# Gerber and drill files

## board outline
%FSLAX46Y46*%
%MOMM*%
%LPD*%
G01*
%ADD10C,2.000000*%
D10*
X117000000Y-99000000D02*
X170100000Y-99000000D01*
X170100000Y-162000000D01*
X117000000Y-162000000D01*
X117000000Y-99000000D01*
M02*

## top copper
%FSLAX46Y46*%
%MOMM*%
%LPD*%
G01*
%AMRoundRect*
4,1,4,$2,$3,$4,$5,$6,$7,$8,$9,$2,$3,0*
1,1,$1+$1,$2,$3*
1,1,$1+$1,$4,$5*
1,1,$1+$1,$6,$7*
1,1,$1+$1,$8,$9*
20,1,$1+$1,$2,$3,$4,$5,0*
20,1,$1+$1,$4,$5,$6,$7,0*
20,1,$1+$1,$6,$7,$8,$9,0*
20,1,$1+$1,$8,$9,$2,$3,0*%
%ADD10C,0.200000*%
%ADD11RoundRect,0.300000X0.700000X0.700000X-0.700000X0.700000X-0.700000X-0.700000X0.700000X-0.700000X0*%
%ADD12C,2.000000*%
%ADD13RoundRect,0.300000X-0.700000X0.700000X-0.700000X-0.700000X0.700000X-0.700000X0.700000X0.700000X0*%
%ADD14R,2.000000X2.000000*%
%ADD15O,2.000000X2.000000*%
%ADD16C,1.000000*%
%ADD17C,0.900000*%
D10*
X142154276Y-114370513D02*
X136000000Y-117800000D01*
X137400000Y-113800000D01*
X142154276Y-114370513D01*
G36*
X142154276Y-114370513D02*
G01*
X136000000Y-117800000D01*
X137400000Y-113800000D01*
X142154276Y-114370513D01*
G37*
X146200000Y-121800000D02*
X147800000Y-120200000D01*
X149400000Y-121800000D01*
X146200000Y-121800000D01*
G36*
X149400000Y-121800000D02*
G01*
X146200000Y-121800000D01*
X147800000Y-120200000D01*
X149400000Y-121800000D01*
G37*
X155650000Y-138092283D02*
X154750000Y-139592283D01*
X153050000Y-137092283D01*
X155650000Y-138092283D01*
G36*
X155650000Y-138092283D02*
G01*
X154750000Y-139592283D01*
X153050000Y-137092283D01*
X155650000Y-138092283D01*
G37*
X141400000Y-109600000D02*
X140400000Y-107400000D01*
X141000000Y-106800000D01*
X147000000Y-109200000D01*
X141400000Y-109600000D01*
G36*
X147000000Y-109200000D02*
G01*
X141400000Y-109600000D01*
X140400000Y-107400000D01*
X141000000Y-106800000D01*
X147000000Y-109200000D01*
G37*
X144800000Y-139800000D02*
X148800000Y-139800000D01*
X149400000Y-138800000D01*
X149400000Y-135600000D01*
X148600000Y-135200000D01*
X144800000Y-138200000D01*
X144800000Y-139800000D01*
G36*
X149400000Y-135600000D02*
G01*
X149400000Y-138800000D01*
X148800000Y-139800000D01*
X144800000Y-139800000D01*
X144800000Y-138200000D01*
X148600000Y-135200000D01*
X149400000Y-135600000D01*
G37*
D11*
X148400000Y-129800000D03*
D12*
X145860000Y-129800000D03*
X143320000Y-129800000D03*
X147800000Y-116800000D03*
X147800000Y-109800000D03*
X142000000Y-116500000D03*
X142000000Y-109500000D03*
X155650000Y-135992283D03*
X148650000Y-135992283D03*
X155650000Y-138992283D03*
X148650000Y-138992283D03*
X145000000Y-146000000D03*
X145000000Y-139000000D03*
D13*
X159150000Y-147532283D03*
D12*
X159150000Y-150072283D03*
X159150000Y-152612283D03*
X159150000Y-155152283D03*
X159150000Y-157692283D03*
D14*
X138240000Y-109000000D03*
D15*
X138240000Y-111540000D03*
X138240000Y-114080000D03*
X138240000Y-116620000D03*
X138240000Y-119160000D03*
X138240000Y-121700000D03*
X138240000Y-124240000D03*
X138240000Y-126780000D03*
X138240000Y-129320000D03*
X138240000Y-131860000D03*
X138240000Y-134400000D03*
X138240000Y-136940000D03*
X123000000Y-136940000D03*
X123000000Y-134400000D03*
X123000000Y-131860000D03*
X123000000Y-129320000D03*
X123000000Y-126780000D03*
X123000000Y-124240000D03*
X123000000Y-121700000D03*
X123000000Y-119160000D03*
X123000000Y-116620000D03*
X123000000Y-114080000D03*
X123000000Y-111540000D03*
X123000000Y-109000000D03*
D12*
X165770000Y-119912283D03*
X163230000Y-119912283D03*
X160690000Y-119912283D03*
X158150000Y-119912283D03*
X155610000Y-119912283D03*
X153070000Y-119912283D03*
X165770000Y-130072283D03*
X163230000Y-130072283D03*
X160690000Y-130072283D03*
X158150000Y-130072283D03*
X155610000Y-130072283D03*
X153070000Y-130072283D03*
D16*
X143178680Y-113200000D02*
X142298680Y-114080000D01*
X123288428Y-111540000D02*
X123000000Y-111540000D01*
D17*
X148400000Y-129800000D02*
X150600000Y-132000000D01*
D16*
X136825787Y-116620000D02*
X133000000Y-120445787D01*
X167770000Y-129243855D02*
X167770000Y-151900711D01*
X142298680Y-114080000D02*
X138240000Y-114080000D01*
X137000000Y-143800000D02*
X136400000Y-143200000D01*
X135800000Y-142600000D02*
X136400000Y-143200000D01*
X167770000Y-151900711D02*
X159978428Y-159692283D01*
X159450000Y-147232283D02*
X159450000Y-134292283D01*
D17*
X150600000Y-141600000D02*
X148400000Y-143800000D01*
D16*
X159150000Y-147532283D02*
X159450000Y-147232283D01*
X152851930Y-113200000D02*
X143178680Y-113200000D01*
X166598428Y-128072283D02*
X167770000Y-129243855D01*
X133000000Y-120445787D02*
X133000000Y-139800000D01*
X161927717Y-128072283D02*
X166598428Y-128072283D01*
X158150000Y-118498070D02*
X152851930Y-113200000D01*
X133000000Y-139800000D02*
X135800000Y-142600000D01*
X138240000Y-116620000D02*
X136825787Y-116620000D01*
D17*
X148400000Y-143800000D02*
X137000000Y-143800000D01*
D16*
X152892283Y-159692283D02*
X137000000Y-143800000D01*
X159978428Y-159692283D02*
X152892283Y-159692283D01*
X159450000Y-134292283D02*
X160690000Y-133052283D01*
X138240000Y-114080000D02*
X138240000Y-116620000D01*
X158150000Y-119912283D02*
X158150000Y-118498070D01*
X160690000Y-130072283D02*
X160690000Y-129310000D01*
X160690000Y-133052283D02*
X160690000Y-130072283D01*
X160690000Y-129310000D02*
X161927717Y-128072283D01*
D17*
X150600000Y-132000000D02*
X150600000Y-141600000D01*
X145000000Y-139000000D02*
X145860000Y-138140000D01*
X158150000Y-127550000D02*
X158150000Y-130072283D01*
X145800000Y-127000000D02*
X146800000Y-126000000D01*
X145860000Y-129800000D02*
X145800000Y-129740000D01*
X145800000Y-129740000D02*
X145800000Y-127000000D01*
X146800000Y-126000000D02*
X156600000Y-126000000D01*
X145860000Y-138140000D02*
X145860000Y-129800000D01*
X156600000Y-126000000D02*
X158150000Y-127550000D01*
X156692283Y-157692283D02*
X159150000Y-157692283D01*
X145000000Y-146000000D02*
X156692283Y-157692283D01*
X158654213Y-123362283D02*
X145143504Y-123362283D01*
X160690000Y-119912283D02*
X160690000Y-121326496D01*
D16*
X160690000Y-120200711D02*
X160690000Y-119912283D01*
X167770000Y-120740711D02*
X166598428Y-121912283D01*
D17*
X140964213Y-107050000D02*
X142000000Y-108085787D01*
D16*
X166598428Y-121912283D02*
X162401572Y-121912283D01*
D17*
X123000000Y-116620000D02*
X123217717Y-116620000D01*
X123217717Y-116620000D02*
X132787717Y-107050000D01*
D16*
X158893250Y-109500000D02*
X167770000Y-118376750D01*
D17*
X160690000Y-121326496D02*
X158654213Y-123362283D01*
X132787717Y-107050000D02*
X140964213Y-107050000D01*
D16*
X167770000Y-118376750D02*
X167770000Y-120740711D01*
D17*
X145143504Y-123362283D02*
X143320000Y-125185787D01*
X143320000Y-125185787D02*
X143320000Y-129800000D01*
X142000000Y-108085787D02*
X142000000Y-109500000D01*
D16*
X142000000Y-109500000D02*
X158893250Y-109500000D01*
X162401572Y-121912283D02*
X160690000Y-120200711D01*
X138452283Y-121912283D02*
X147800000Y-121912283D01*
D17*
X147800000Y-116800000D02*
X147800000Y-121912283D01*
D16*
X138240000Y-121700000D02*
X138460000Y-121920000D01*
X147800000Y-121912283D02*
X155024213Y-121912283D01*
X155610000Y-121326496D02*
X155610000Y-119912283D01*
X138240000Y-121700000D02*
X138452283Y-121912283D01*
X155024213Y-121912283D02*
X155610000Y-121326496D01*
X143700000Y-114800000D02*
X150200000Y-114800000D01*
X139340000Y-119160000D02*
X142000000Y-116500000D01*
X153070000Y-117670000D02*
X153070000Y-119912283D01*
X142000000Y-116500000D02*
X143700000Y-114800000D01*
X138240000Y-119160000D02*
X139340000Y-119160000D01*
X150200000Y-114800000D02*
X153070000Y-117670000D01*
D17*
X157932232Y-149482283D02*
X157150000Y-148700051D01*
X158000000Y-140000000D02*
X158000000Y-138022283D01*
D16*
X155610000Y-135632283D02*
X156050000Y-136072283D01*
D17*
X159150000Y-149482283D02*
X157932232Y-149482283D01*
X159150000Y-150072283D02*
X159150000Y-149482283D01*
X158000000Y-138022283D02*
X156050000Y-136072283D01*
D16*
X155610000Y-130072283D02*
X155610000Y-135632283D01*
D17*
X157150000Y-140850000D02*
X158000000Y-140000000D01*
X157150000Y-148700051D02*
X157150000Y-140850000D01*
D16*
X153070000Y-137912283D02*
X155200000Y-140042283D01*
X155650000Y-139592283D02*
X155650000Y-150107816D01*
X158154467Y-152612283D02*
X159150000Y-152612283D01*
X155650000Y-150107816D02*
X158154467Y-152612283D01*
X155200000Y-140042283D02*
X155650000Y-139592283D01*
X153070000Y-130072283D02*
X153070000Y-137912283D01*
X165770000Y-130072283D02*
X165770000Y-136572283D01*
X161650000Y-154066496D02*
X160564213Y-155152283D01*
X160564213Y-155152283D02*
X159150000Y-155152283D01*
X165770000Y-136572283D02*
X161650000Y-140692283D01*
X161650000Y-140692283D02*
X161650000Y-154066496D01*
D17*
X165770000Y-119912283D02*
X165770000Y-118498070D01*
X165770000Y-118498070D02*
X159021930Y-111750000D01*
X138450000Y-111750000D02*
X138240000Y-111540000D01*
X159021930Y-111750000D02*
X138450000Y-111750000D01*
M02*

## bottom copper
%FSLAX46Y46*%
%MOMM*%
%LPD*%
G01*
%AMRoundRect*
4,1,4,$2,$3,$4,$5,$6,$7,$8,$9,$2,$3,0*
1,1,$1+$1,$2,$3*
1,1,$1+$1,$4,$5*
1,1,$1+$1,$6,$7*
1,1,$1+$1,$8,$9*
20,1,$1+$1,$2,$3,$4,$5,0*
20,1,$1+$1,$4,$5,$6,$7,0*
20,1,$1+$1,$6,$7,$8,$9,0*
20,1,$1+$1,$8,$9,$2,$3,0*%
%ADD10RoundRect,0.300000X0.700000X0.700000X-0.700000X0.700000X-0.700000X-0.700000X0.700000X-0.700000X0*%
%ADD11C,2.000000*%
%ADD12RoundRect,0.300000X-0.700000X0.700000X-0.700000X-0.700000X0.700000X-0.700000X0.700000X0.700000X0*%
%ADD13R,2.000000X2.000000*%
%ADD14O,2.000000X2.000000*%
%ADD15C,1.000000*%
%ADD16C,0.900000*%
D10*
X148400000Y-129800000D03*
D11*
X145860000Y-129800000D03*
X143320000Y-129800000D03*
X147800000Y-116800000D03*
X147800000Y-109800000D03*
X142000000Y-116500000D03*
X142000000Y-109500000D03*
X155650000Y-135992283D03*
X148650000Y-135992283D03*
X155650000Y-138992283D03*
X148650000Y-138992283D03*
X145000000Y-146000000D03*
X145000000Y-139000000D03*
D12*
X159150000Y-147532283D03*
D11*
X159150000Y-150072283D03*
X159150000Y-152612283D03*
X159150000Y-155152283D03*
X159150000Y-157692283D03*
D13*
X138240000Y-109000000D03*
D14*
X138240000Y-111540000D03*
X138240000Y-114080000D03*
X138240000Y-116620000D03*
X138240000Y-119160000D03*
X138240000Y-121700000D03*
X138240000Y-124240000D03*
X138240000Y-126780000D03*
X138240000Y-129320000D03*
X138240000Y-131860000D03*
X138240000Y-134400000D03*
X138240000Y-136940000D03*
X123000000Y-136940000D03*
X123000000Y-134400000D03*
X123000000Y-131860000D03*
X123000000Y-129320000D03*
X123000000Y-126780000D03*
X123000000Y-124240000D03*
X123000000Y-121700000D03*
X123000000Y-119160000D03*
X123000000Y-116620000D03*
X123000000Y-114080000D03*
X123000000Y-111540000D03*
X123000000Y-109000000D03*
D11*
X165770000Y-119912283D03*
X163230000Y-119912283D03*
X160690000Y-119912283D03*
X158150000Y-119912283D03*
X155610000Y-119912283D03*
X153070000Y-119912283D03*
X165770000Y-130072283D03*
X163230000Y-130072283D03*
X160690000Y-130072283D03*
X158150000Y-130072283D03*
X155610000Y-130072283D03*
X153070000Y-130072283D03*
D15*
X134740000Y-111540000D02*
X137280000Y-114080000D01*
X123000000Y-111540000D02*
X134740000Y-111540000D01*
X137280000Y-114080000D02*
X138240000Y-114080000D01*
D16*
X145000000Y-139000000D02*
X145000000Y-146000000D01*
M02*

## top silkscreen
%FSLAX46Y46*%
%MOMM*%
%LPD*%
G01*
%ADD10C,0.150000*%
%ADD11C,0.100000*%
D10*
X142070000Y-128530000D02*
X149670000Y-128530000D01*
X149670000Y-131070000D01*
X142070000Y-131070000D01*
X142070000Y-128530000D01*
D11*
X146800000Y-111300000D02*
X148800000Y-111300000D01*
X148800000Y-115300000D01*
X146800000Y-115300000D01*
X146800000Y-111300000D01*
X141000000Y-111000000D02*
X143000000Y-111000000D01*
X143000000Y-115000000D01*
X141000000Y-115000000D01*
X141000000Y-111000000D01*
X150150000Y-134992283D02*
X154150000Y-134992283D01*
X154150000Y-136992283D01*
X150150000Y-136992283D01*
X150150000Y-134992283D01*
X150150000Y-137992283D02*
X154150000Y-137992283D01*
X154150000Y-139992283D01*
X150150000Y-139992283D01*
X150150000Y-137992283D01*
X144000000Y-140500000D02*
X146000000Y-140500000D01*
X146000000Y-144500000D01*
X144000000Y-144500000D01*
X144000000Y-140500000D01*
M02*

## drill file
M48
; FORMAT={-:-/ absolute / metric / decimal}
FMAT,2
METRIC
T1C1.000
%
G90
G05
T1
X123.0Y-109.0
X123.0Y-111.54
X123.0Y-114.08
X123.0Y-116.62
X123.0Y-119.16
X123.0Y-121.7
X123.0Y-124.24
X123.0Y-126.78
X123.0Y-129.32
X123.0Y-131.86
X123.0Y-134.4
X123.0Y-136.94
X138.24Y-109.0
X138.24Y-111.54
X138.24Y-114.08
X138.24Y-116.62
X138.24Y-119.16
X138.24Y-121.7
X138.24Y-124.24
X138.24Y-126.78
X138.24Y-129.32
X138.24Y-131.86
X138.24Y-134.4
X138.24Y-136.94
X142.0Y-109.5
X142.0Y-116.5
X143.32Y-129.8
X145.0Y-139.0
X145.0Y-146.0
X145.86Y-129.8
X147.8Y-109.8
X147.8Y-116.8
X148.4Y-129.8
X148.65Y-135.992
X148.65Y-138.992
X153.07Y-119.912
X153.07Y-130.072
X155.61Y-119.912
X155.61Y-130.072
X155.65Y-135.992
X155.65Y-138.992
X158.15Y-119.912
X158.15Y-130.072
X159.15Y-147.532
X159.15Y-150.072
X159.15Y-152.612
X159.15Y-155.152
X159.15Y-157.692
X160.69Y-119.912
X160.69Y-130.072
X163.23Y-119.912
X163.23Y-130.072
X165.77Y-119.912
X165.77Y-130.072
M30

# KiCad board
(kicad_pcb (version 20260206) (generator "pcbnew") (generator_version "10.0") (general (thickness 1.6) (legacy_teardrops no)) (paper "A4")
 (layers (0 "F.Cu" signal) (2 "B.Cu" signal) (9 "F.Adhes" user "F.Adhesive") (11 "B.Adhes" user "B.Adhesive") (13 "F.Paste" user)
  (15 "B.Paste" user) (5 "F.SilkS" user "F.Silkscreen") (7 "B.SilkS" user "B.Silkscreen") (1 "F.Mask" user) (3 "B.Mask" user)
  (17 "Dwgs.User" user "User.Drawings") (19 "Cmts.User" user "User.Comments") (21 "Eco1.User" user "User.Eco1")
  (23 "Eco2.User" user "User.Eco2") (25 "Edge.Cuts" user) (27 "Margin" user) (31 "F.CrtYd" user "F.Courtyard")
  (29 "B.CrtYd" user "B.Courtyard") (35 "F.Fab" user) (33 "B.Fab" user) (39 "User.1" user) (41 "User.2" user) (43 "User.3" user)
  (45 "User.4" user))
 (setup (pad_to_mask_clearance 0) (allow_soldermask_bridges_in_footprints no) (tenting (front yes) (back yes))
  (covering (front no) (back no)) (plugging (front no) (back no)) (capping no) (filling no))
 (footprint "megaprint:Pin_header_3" (layer "F.Cu") (at 145.86 129.8 180)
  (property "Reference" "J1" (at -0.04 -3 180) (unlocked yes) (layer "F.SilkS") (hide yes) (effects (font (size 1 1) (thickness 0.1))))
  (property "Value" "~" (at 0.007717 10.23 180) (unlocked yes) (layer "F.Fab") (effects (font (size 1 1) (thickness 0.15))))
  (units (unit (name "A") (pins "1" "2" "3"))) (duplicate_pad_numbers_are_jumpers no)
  (fp_rect (start -3.81 -1.27) (end 3.79 1.27) (stroke (width 0.15) (type default)) (fill no) (layer "F.SilkS"))
  (pad "1" thru_hole roundrect (at -2.54 0 180) (size 2 2) (drill 1) (layers "*.Cu" "*.Mask") (remove_unused_layers no)
   (roundrect_rratio 0.15) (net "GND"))
  (pad "2" thru_hole circle (at 0 0 180) (size 2 2) (drill 1) (layers "*.Cu" "*.Mask") (remove_unused_layers no) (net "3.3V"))
  (pad "3" thru_hole circle (at 2.54 0 180) (size 2 2) (drill 1) (layers "*.Cu" "*.Mask") (remove_unused_layers no) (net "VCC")))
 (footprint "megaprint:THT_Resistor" (layer "F.Cu") (at 147.8 113.3 90)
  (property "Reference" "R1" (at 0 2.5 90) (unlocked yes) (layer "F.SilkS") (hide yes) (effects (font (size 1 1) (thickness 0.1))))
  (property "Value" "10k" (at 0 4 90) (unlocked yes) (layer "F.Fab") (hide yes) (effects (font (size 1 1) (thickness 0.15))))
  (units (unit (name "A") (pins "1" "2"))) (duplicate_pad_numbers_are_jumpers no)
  (fp_rect (start -2 -1) (end 2 1) (stroke (width 0.1) (type default)) (fill no) (layer "F.SilkS"))
  (pad "1" thru_hole circle (at -3.5 0 90) (size 2 2) (drill 1) (layers "*.Cu" "*.Mask") (remove_unused_layers no) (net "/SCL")
   (thermal_bridge_angle 90))
  (pad "2" thru_hole circle (at 3.5 0 90) (size 2 2) (drill 1) (layers "*.Cu" "*.Mask") (remove_unused_layers no) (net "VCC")
   (thermal_bridge_angle 90)))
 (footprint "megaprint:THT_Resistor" (layer "F.Cu") (at 142 113 90)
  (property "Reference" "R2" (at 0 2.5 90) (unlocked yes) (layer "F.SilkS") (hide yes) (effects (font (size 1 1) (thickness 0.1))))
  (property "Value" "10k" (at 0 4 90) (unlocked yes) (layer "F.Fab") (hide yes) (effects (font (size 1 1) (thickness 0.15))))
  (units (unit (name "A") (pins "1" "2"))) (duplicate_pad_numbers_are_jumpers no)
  (fp_rect (start -2 -1) (end 2 1) (stroke (width 0.1) (type default)) (fill no) (layer "F.SilkS"))
  (pad "1" thru_hole circle (at -3.5 0 90) (size 2 2) (drill 1) (layers "*.Cu" "*.Mask") (remove_unused_layers no) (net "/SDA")
   (thermal_bridge_angle 90))
  (pad "2" thru_hole circle (at 3.5 0 90) (size 2 2) (drill 1) (layers "*.Cu" "*.Mask") (remove_unused_layers no) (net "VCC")
   (thermal_bridge_angle 90)))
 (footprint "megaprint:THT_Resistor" (layer "F.Cu") (at 152.15 135.992283 180)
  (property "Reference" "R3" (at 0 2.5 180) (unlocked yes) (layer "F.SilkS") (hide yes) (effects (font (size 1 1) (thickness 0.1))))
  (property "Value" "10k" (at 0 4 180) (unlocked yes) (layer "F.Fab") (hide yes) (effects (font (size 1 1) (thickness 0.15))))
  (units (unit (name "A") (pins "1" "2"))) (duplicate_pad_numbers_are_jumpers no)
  (fp_rect (start -2 -1) (end 2 1) (stroke (width 0.1) (type default)) (fill no) (layer "F.SilkS"))
  (pad "1" thru_hole circle (at -3.5 0 180) (size 2 2) (drill 1) (layers "*.Cu" "*.Mask") (remove_unused_layers no) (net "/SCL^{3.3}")
   (thermal_bridge_angle 90))
  (pad "2" thru_hole circle (at 3.5 0 180) (size 2 2) (drill 1) (layers "*.Cu" "*.Mask") (remove_unused_layers no) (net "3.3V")
   (thermal_bridge_angle 90)))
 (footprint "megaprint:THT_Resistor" (layer "F.Cu") (at 152.15 138.992283 180)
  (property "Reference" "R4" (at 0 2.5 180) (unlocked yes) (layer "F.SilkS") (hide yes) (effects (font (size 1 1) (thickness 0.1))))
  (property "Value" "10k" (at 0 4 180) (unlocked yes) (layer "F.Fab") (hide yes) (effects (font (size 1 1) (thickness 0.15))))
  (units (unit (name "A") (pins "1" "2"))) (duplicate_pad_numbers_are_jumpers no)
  (fp_rect (start -2 -1) (end 2 1) (stroke (width 0.1) (type default)) (fill no) (layer "F.SilkS"))
  (pad "1" thru_hole circle (at -3.5 0 180) (size 2 2) (drill 1) (layers "*.Cu" "*.Mask") (remove_unused_layers no) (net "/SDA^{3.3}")
   (thermal_bridge_angle 90))
  (pad "2" thru_hole circle (at 3.5 0 180) (size 2 2) (drill 1) (layers "*.Cu" "*.Mask") (remove_unused_layers no) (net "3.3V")
   (thermal_bridge_angle 90)))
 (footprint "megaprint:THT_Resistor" (layer "F.Cu") (at 145 142.5 90)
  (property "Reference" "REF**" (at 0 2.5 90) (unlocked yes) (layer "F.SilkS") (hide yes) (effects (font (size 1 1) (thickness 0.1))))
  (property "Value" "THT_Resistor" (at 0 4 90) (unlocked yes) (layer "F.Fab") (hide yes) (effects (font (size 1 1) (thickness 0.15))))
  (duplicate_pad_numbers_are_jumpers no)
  (fp_rect (start -2 -1) (end 2 1) (stroke (width 0.1) (type default)) (fill no) (layer "F.SilkS"))
  (pad "1" thru_hole circle (at -3.5 0 90) (size 2 2) (drill 1) (layers "*.Cu" "*.Mask") (remove_unused_layers no) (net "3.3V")
   (thermal_bridge_angle 90))
  (pad "2" thru_hole circle (at 3.5 0 90) (size 2 2) (drill 1) (layers "*.Cu" "*.Mask") (remove_unused_layers no) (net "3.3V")
   (thermal_bridge_angle 90)))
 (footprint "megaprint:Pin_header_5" (layer "B.Cu") (at 159.15 152.612283 -90)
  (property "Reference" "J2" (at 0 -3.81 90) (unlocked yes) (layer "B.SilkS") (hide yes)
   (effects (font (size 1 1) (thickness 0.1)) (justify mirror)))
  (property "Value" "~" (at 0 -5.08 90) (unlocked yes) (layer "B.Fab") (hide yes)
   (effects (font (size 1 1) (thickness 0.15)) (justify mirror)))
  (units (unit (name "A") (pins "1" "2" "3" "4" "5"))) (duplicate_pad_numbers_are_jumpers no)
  (pad "1" thru_hole roundrect (at -5.08 0 270) (size 2 2) (drill 1) (layers "*.Cu" "*.Mask") (remove_unused_layers no)
   (roundrect_rratio 0.15) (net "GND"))
  (pad "2" thru_hole circle (at -2.54 0 270) (size 2 2) (drill 1) (layers "*.Cu" "*.Mask") (remove_unused_layers no) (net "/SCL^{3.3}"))
  (pad "3" thru_hole circle (at 0 0 270) (size 2 2) (drill 1) (layers "*.Cu" "*.Mask") (remove_unused_layers no) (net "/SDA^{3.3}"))
  (pad "4" thru_hole circle (at 2.54 0 270) (size 2 2) (drill 1) (layers "*.Cu" "*.Mask") (remove_unused_layers no) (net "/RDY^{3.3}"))
  (pad "5" thru_hole circle (at 5.08 0 270) (size 2 2) (drill 1) (layers "*.Cu" "*.Mask") (remove_unused_layers no) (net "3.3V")))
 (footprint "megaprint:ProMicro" (layer "B.Cu") (at 130.62 120.43 180)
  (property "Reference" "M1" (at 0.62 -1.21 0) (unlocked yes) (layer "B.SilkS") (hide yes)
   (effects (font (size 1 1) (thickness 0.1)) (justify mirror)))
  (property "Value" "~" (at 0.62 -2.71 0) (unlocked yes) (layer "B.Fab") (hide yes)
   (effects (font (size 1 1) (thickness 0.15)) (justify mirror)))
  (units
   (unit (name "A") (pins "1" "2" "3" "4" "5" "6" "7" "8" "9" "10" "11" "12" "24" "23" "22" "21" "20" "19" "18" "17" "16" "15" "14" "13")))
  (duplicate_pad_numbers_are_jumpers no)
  (pad "1" thru_hole rect (at -7.62 11.43) (size 2 2) (drill 1) (layers "*.Cu" "*.Mask") (remove_unused_layers no)
   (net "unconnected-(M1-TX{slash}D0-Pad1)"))
  (pad "2" thru_hole oval (at -7.62 8.89) (size 2 2) (drill 1) (layers "*.Cu" "*.Mask") (remove_unused_layers no) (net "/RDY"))
  (pad "3" thru_hole oval (at -7.62 6.35) (size 2 2) (drill 1) (layers "*.Cu" "*.Mask") (remove_unused_layers no) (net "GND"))
  (pad "4" thru_hole oval (at -7.62 3.81) (size 2 2) (drill 1) (layers "*.Cu" "*.Mask") (remove_unused_layers no) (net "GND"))
  (pad "5" thru_hole oval (at -7.62 1.27) (size 2 2) (drill 1) (layers "*.Cu" "*.Mask") (remove_unused_layers no) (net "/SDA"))
  (pad "6" thru_hole oval (at -7.62 -1.27) (size 2 2) (drill 1) (layers "*.Cu" "*.Mask") (remove_unused_layers no) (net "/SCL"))
  (pad "7" thru_hole oval (at -7.62 -3.81) (size 2 2) (drill 1) (layers "*.Cu" "*.Mask") (remove_unused_layers no)
   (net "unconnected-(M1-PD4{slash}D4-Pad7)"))
  (pad "8" thru_hole oval (at -7.62 -6.35) (size 2 2) (drill 1) (layers "*.Cu" "*.Mask") (remove_unused_layers no)
   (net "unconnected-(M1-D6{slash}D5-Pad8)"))
  (pad "9" thru_hole oval (at -7.62 -8.89) (size 2 2) (drill 1) (layers "*.Cu" "*.Mask") (remove_unused_layers no)
   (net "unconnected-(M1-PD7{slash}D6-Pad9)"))
  (pad "10" thru_hole oval (at -7.62 -11.43) (size 2 2) (drill 1) (layers "*.Cu" "*.Mask") (remove_unused_layers no)
   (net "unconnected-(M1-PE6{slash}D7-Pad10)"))
  (pad "11" thru_hole oval (at -7.62 -13.97) (size 2 2) (drill 1) (layers "*.Cu" "*.Mask") (remove_unused_layers no)
   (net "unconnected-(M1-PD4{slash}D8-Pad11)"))
  (pad "12" thru_hole oval (at -7.62 -16.51) (size 2 2) (drill 1) (layers "*.Cu" "*.Mask") (remove_unused_layers no)
   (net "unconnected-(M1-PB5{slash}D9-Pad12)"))
  (pad "13" thru_hole oval (at 7.62 -16.51) (size 2 2) (drill 1) (layers "*.Cu" "*.Mask") (remove_unused_layers no)
   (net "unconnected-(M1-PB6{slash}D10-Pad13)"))
  (pad "14" thru_hole oval (at 7.62 -13.97) (size 2 2) (drill 1) (layers "*.Cu" "*.Mask") (remove_unused_layers no)
   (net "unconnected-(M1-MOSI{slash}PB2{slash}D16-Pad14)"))
  (pad "15" thru_hole oval (at 7.62 -11.43) (size 2 2) (drill 1) (layers "*.Cu" "*.Mask") (remove_unused_layers no)
   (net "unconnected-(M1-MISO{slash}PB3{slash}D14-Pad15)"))
  (pad "16" thru_hole oval (at 7.62 -8.89) (size 2 2) (drill 1) (layers "*.Cu" "*.Mask") (remove_unused_layers no)
   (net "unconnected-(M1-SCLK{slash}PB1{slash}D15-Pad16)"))
  (pad "17" thru_hole oval (at 7.62 -6.35) (size 2 2) (drill 1) (layers "*.Cu" "*.Mask") (remove_unused_layers no)
   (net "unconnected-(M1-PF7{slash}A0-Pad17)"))
  (pad "18" thru_hole oval (at 7.62 -3.81) (size 2 2) (drill 1) (layers "*.Cu" "*.Mask") (remove_unused_layers no)
   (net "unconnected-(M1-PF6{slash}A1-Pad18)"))
  (pad "19" thru_hole oval (at 7.62 -1.27) (size 2 2) (drill 1) (layers "*.Cu" "*.Mask") (remove_unused_layers no)
   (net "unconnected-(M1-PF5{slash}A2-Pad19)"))
  (pad "20" thru_hole oval (at 7.62 1.27) (size 2 2) (drill 1) (layers "*.Cu" "*.Mask") (remove_unused_layers no)
   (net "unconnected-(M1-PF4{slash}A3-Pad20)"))
  (pad "21" thru_hole oval (at 7.62 3.81) (size 2 2) (drill 1) (layers "*.Cu" "*.Mask") (remove_unused_layers no) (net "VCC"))
  (pad "22" thru_hole oval (at 7.62 6.35) (size 2 2) (drill 1) (layers "*.Cu" "*.Mask") (remove_unused_layers no)
   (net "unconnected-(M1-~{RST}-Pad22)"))
  (pad "23" thru_hole oval (at 7.62 8.89) (size 2 2) (drill 1) (layers "*.Cu" "*.Mask") (remove_unused_layers no) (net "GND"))
  (pad "24" thru_hole oval (at 7.62 11.43) (size 2 2) (drill 1) (layers "*.Cu" "*.Mask") (remove_unused_layers no)
   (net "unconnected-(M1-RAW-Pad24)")))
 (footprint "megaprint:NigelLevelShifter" (layer "B.Cu") (at 159.4125 124.992283 180)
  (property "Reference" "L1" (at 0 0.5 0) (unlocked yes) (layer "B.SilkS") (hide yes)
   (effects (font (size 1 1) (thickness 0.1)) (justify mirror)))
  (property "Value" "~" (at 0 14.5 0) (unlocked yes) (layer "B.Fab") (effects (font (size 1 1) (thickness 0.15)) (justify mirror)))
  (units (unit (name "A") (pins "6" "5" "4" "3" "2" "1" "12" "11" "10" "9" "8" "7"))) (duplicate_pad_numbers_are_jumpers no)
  (pad "1" thru_hole circle (at -6.3575 5.08 180) (size 2 2) (drill 1) (layers "*.Cu" "*.Mask") (remove_unused_layers no) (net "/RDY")
   (thermal_bridge_angle 90))
  (pad "2" thru_hole circle (at -3.8175 5.08 180) (size 2 2) (drill 1) (layers "*.Cu" "*.Mask") (remove_unused_layers no)
   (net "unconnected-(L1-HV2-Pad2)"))
  (pad "3" thru_hole circle (at -1.2775 5.08 180) (size 2 2) (drill 1) (layers "*.Cu" "*.Mask") (remove_unused_layers no) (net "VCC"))
  (pad "4" thru_hole circle (at 1.2625 5.08 180) (size 2 2) (drill 1) (layers "*.Cu" "*.Mask") (remove_unused_layers no) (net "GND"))
  (pad "5" thru_hole circle (at 3.8025 5.08 180) (size 2 2) (drill 1) (layers "*.Cu" "*.Mask") (remove_unused_layers no) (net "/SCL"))
  (pad "6" thru_hole circle (at 6.3425 5.08 180) (size 2 2) (drill 1) (layers "*.Cu" "*.Mask") (remove_unused_layers no) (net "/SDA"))
  (pad "7" thru_hole circle (at -6.3575 -5.08 180) (size 2 2) (drill 1) (layers "*.Cu" "*.Mask") (remove_unused_layers no)
   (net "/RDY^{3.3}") (thermal_bridge_angle 90))
  (pad "8" thru_hole circle (at -3.8175 -5.08 180) (size 2 2) (drill 1) (layers "*.Cu" "*.Mask") (remove_unused_layers no)
   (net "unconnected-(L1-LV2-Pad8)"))
  (pad "9" thru_hole circle (at -1.2775 -5.08 180) (size 2 2) (drill 1) (layers "*.Cu" "*.Mask") (remove_unused_layers no) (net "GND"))
  (pad "10" thru_hole circle (at 1.2625 -5.08 180) (size 2 2) (drill 1) (layers "*.Cu" "*.Mask") (remove_unused_layers no) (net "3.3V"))
  (pad "11" thru_hole circle (at 3.8025 -5.08 180) (size 2 2) (drill 1) (layers "*.Cu" "*.Mask") (remove_unused_layers no)
   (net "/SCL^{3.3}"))
  (pad "12" thru_hole circle (at 6.3425 -5.08 180) (size 2 2) (drill 1) (layers "*.Cu" "*.Mask") (remove_unused_layers no)
   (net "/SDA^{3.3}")))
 (gr_poly
  (pts (xy 142.154276 114.370513) (xy 136 117.8) (xy 137.4 113.8)) (stroke (width 0.2) (type solid)) (fill yes) (layer "F.Cu") (net "GND"))
 (gr_poly (pts (xy 146.2 121.8) (xy 147.8 120.2) (xy 149.4 121.8)) (stroke (width 0.2) (type solid)) (fill yes) (layer "F.Cu") (net "/SCL"))
 (gr_poly
  (pts (xy 155.65 138.092283) (xy 154.75 139.592283) (xy 153.05 137.092283)) (stroke (width 0.2) (type solid)) (fill yes) (layer "F.Cu")
  (net "/SDA^{3.3}"))
 (gr_poly
  (pts (xy 141.4 109.6) (xy 140.4 107.4) (xy 141 106.8) (xy 147 109.2)) (stroke (width 0.2) (type solid)) (fill yes) (layer "F.Cu")
  (net "VCC"))
 (gr_poly
  (pts (xy 144.8 139.8) (xy 148.8 139.8) (xy 149.4 138.8) (xy 149.4 135.6) (xy 148.6 135.2) (xy 144.8 138.2))
  (stroke (width 0.2) (type solid)) (fill yes) (layer "F.Cu") (net "3.3V"))
 (gr_rect (start 117 99) (end 170.1 162) (stroke (width 2) (type solid)) (fill no) (layer "Edge.Cuts"))
 (segment (start 143.17868 113.2) (end 142.29868 114.08) (width 1) (layer "F.Cu") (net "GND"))
 (segment (start 123.288428 111.54) (end 123 111.54) (width 1) (layer "F.Cu") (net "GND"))
 (segment (start 148.4 129.8) (end 150.6 132) (width 0.9) (layer "F.Cu") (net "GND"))
 (segment (start 136.825787 116.62) (end 133 120.445787) (width 1) (layer "F.Cu") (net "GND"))
 (segment (start 167.77 129.243855) (end 167.77 151.900711) (width 1) (layer "F.Cu") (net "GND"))
 (segment (start 142.29868 114.08) (end 138.24 114.08) (width 1) (layer "F.Cu") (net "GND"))
 (segment (start 137 143.8) (end 136.4 143.2) (width 1) (layer "F.Cu") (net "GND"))
 (segment (start 135.8 142.6) (end 136.4 143.2) (width 1) (layer "F.Cu") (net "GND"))
 (segment (start 167.77 151.900711) (end 159.978428 159.692283) (width 1) (layer "F.Cu") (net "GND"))
 (segment (start 159.45 147.232283) (end 159.45 134.292283) (width 1) (layer "F.Cu") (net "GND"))
 (segment (start 150.6 141.6) (end 148.4 143.8) (width 0.9) (layer "F.Cu") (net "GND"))
 (segment (start 159.15 147.532283) (end 159.45 147.232283) (width 1) (layer "F.Cu") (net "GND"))
 (segment (start 152.85193 113.2) (end 143.17868 113.2) (width 1) (layer "F.Cu") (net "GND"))
 (segment (start 166.598428 128.072283) (end 167.77 129.243855) (width 1) (layer "F.Cu") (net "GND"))
 (segment (start 133 120.445787) (end 133 139.8) (width 1) (layer "F.Cu") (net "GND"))
 (segment (start 161.927717 128.072283) (end 166.598428 128.072283) (width 1) (layer "F.Cu") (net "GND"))
 (segment (start 158.15 118.49807) (end 152.85193 113.2) (width 1) (layer "F.Cu") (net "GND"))
 (segment (start 133 139.8) (end 135.8 142.6) (width 1) (layer "F.Cu") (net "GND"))
 (segment (start 138.24 116.62) (end 136.825787 116.62) (width 1) (layer "F.Cu") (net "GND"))
 (segment (start 148.4 143.8) (end 137 143.8) (width 0.9) (layer "F.Cu") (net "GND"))
 (segment (start 152.892283 159.692283) (end 137 143.8) (width 1) (layer "F.Cu") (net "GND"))
 (segment (start 159.978428 159.692283) (end 152.892283 159.692283) (width 1) (layer "F.Cu") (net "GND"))
 (segment (start 159.45 134.292283) (end 160.69 133.052283) (width 1) (layer "F.Cu") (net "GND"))
 (segment (start 138.24 114.08) (end 138.24 116.62) (width 1) (layer "F.Cu") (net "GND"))
 (segment (start 158.15 119.912283) (end 158.15 118.49807) (width 1) (layer "F.Cu") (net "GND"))
 (segment (start 160.69 130.072283) (end 160.69 129.31) (width 1) (layer "F.Cu") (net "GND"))
 (segment (start 160.69 133.052283) (end 160.69 130.072283) (width 1) (layer "F.Cu") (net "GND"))
 (segment (start 160.69 129.31) (end 161.927717 128.072283) (width 1) (layer "F.Cu") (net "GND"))
 (segment (start 150.6 132) (end 150.6 141.6) (width 0.9) (layer "F.Cu") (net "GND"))
 (segment (start 134.74 111.54) (end 137.28 114.08) (width 1) (layer "B.Cu") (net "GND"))
 (segment (start 123 111.54) (end 134.74 111.54) (width 1) (layer "B.Cu") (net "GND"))
 (segment (start 137.28 114.08) (end 138.24 114.08) (width 1) (layer "B.Cu") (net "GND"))
 (segment (start 145 139) (end 145.86 138.14) (width 0.9) (layer "F.Cu") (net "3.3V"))
 (segment (start 158.15 127.55) (end 158.15 130.072283) (width 0.9) (layer "F.Cu") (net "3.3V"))
 (segment (start 145.8 127) (end 146.8 126) (width 0.9) (layer "F.Cu") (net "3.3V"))
 (segment (start 145.86 129.8) (end 145.8 129.74) (width 0.9) (layer "F.Cu") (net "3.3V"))
 (segment (start 145.8 129.74) (end 145.8 127) (width 0.9) (layer "F.Cu") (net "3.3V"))
 (segment (start 146.8 126) (end 156.6 126) (width 0.9) (layer "F.Cu") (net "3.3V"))
 (segment (start 145.86 138.14) (end 145.86 129.8) (width 0.9) (layer "F.Cu") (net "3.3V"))
 (segment (start 156.6 126) (end 158.15 127.55) (width 0.9) (layer "F.Cu") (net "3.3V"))
 (segment (start 156.692283 157.692283) (end 159.15 157.692283) (width 0.9) (layer "F.Cu") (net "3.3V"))
 (segment (start 145 146) (end 156.692283 157.692283) (width 0.9) (layer "F.Cu") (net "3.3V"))
 (segment (start 145 139) (end 145 146) (width 0.9) (layer "B.Cu") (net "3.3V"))
 (segment (start 158.654213 123.362283) (end 145.143504 123.362283) (width 0.9) (layer "F.Cu") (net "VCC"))
 (segment (start 160.69 119.912283) (end 160.69 121.326496) (width 0.9) (layer "F.Cu") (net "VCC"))
 (segment (start 160.69 120.200711) (end 160.69 119.912283) (width 1) (layer "F.Cu") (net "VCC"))
 (segment (start 167.77 120.740711) (end 166.598428 121.912283) (width 1) (layer "F.Cu") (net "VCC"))
 (segment (start 140.964213 107.05) (end 142 108.085787) (width 0.9) (layer "F.Cu") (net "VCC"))
 (segment (start 166.598428 121.912283) (end 162.401572 121.912283) (width 1) (layer "F.Cu") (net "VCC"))
 (segment (start 123 116.62) (end 123.217717 116.62) (width 0.9) (layer "F.Cu") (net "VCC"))
 (segment (start 123.217717 116.62) (end 132.787717 107.05) (width 0.9) (layer "F.Cu") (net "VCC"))
 (segment (start 158.89325 109.5) (end 167.77 118.37675) (width 1) (layer "F.Cu") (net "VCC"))
 (segment (start 160.69 121.326496) (end 158.654213 123.362283) (width 0.9) (layer "F.Cu") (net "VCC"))
 (segment (start 132.787717 107.05) (end 140.964213 107.05) (width 0.9) (layer "F.Cu") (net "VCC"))
 (segment (start 167.77 118.37675) (end 167.77 120.740711) (width 1) (layer "F.Cu") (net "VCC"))
 (segment (start 145.143504 123.362283) (end 143.32 125.185787) (width 0.9) (layer "F.Cu") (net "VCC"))
 (segment (start 143.32 125.185787) (end 143.32 129.8) (width 0.9) (layer "F.Cu") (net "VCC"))
 (segment (start 142 108.085787) (end 142 109.5) (width 0.9) (layer "F.Cu") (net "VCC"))
 (segment (start 142 109.5) (end 158.89325 109.5) (width 1) (layer "F.Cu") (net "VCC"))
 (segment (start 162.401572 121.912283) (end 160.69 120.200711) (width 1) (layer "F.Cu") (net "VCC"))
 (segment (start 138.452283 121.912283) (end 147.8 121.912283) (width 1) (layer "F.Cu") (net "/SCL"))
 (segment (start 147.8 116.8) (end 147.8 121.912283) (width 0.9) (layer "F.Cu") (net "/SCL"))
 (segment (start 138.24 121.7) (end 138.46 121.92) (width 1) (layer "F.Cu") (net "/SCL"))
 (segment (start 147.8 121.912283) (end 155.024213 121.912283) (width 1) (layer "F.Cu") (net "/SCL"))
 (segment (start 155.61 121.326496) (end 155.61 119.912283) (width 1) (layer "F.Cu") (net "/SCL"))
 (segment (start 138.24 121.7) (end 138.452283 121.912283) (width 1) (layer "F.Cu") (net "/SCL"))
 (segment (start 155.024213 121.912283) (end 155.61 121.326496) (width 1) (layer "F.Cu") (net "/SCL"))
 (segment (start 143.7 114.8) (end 150.2 114.8) (width 1) (layer "F.Cu") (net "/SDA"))
 (segment (start 139.34 119.16) (end 142 116.5) (width 1) (layer "F.Cu") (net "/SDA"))
 (segment (start 153.07 117.67) (end 153.07 119.912283) (width 1) (layer "F.Cu") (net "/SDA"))
 (segment (start 142 116.5) (end 143.7 114.8) (width 1) (layer "F.Cu") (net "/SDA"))
 (segment (start 138.24 119.16) (end 139.34 119.16) (width 1) (layer "F.Cu") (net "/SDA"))
 (segment (start 150.2 114.8) (end 153.07 117.67) (width 1) (layer "F.Cu") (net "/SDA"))
 (segment (start 157.932232 149.482283) (end 157.15 148.700051) (width 0.9) (layer "F.Cu") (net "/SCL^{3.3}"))
 (segment (start 158 140) (end 158 138.022283) (width 0.9) (layer "F.Cu") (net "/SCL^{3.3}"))
 (segment (start 155.61 135.632283) (end 156.05 136.072283) (width 1) (layer "F.Cu") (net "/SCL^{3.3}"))
 (segment (start 159.15 149.482283) (end 157.932232 149.482283) (width 0.9) (layer "F.Cu") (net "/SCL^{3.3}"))
 (segment (start 159.15 150.072283) (end 159.15 149.482283) (width 0.9) (layer "F.Cu") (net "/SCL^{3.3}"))
 (segment (start 158 138.022283) (end 156.05 136.072283) (width 0.9) (layer "F.Cu") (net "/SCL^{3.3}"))
 (segment (start 155.61 130.072283) (end 155.61 135.632283) (width 1) (layer "F.Cu") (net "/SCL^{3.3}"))
 (segment (start 157.15 140.85) (end 158 140) (width 0.9) (layer "F.Cu") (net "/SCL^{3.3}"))
 (segment (start 157.15 148.700051) (end 157.15 140.85) (width 0.9) (layer "F.Cu") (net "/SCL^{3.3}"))
 (segment (start 153.07 137.912283) (end 155.2 140.042283) (width 1) (layer "F.Cu") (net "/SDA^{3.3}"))
 (segment (start 155.65 139.592283) (end 155.65 150.107816) (width 1) (layer "F.Cu") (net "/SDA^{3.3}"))
 (segment (start 158.154467 152.612283) (end 159.15 152.612283) (width 1) (layer "F.Cu") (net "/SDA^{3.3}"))
 (segment (start 155.65 150.107816) (end 158.154467 152.612283) (width 1) (layer "F.Cu") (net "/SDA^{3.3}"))
 (segment (start 155.2 140.042283) (end 155.65 139.592283) (width 1) (layer "F.Cu") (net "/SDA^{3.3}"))
 (segment (start 153.07 130.072283) (end 153.07 137.912283) (width 1) (layer "F.Cu") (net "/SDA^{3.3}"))
 (segment (start 165.77 130.072283) (end 165.77 136.572283) (width 1) (layer "F.Cu") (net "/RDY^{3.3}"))
 (segment (start 161.65 154.066496) (end 160.564213 155.152283) (width 1) (layer "F.Cu") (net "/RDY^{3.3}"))
 (segment (start 160.564213 155.152283) (end 159.15 155.152283) (width 1) (layer "F.Cu") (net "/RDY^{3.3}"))
 (segment (start 165.77 136.572283) (end 161.65 140.692283) (width 1) (layer "F.Cu") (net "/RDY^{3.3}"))
 (segment (start 161.65 140.692283) (end 161.65 154.066496) (width 1) (layer "F.Cu") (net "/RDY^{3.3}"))
 (segment (start 165.77 119.912283) (end 165.77 118.49807) (width 0.9) (layer "F.Cu") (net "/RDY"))
 (segment (start 165.77 118.49807) (end 159.02193 111.75) (width 0.9) (layer "F.Cu") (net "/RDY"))
 (segment (start 138.45 111.75) (end 138.24 111.54) (width 0.9) (layer "F.Cu") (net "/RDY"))
 (segment (start 159.02193 111.75) (end 138.45 111.75) (width 0.9) (layer "F.Cu") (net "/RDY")))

